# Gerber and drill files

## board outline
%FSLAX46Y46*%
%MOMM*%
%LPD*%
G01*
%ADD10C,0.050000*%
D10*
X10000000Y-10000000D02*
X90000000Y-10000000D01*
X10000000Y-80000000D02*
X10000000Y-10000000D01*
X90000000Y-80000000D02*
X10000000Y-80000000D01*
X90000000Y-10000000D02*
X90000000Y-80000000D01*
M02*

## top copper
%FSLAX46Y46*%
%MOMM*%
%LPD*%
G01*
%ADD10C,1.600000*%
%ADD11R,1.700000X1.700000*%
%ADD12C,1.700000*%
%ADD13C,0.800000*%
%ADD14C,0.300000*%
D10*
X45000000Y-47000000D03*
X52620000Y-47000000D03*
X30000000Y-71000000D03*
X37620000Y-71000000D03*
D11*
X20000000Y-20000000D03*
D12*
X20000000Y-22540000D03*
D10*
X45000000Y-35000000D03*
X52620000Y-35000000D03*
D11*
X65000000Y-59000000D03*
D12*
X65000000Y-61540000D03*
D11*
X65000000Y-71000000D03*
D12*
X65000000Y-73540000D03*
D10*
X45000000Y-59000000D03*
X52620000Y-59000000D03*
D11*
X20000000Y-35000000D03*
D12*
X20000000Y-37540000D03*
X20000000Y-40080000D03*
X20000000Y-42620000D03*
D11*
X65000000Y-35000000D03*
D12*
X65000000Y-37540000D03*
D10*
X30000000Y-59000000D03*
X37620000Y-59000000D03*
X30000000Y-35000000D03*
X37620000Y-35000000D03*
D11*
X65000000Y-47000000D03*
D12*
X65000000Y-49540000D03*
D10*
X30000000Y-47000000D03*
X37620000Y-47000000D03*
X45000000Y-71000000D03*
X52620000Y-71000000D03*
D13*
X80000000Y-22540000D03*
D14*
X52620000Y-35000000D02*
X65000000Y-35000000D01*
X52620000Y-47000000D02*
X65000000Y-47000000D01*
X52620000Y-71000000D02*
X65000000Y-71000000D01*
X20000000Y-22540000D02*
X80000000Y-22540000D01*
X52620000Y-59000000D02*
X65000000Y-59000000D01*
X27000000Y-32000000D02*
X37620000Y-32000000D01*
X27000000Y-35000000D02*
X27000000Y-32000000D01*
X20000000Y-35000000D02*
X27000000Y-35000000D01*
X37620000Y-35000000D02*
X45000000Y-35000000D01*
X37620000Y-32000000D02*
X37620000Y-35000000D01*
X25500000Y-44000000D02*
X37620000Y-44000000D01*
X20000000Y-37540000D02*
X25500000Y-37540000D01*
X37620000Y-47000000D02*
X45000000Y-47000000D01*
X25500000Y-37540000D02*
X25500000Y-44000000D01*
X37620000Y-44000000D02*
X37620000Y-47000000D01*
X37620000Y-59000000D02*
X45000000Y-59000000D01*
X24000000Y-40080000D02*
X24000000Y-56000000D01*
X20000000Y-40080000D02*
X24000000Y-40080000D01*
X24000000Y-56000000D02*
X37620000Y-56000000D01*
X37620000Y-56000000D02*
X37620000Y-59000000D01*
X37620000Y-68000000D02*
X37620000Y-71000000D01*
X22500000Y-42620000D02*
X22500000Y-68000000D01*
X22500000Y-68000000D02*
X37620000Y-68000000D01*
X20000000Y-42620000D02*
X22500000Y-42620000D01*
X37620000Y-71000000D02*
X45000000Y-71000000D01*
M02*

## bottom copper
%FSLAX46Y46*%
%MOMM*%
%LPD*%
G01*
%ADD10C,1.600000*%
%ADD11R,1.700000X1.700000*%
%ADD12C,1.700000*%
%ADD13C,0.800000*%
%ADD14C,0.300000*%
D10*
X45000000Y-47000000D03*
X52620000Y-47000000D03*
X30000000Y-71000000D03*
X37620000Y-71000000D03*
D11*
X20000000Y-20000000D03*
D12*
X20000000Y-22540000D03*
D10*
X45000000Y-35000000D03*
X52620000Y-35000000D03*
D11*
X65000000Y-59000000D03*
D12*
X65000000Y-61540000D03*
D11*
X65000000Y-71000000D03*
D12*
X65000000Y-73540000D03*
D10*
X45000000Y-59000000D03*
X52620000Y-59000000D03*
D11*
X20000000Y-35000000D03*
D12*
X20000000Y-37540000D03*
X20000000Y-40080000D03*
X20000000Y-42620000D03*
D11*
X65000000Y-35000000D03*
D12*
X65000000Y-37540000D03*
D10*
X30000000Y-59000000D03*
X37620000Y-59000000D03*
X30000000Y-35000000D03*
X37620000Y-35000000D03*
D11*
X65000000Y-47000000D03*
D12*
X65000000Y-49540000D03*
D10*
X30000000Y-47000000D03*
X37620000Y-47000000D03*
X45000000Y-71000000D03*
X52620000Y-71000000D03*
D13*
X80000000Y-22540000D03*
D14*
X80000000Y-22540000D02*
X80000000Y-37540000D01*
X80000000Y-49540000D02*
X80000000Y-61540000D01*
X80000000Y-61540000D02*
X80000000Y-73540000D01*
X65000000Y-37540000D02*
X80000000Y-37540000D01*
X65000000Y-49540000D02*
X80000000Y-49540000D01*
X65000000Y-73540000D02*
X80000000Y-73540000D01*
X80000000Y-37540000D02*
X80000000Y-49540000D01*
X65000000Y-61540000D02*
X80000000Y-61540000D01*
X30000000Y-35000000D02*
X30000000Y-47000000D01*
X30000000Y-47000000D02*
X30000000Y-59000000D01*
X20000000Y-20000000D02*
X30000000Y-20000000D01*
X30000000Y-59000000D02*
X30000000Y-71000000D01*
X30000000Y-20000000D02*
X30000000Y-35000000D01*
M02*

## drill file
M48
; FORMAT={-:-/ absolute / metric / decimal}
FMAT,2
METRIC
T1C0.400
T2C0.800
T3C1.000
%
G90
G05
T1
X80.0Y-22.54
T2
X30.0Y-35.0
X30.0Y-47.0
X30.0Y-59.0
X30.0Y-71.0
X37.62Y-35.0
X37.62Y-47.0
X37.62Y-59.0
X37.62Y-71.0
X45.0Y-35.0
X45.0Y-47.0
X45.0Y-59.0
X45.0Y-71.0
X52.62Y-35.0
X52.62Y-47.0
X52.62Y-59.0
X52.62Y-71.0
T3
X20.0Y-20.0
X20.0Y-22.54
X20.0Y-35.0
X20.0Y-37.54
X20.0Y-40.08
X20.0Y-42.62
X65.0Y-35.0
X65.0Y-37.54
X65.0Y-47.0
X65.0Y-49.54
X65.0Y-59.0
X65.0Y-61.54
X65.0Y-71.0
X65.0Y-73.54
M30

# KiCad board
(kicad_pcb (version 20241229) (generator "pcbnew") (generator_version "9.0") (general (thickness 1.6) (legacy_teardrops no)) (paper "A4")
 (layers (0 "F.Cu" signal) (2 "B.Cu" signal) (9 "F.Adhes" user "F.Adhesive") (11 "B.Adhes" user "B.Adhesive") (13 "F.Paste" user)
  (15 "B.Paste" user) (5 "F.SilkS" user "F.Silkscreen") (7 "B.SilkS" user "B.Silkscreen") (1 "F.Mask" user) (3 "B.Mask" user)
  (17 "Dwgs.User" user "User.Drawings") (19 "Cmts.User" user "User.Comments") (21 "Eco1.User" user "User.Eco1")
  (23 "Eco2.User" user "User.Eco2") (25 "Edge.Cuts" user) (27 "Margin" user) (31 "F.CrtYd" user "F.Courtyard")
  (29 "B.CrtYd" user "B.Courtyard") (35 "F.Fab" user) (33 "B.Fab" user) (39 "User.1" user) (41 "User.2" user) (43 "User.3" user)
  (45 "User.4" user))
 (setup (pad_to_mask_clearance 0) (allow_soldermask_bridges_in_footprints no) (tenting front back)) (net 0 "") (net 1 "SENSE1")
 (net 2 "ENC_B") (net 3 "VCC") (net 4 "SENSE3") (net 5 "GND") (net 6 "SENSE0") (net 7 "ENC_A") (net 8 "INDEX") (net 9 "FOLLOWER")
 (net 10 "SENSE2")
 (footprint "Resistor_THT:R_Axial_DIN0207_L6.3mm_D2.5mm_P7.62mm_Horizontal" (layer "F.Cu") (at 45 47)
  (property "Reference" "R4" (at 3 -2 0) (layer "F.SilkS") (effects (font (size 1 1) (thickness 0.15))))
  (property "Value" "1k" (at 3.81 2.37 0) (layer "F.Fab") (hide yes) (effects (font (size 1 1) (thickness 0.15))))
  (pad "1" thru_hole circle (at 0 0) (size 1.6 1.6) (drill 0.8) (layers "*.Cu" "*.Mask") (remove_unused_layers no) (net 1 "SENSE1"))
  (pad "2" thru_hole circle (at 7.62 0) (size 1.6 1.6) (drill 0.8) (layers "*.Cu" "*.Mask") (remove_unused_layers no) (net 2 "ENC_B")))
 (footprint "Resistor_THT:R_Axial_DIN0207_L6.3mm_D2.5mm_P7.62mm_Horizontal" (layer "F.Cu") (at 30 71)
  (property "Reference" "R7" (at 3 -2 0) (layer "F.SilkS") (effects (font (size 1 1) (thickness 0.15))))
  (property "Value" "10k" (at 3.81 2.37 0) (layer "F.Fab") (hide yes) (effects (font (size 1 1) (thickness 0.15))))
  (pad "1" thru_hole circle (at 0 0) (size 1.6 1.6) (drill 0.8) (layers "*.Cu" "*.Mask") (remove_unused_layers no) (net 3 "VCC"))
  (pad "2" thru_hole circle (at 7.62 0) (size 1.6 1.6) (drill 0.8) (layers "*.Cu" "*.Mask") (remove_unused_layers no) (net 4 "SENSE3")))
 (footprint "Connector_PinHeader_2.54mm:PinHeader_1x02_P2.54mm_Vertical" (layer "F.Cu") (at 20 20)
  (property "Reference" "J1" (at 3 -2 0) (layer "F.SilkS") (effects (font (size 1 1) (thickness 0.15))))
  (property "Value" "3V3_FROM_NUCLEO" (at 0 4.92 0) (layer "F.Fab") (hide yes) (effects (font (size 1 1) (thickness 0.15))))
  (pad "1" thru_hole rect (at 0 0) (size 1.7 1.7) (drill 1) (layers "*.Cu" "*.Mask") (remove_unused_layers no) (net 3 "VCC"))
  (pad "2" thru_hole circle (at 0 2.54) (size 1.7 1.7) (drill 1) (layers "*.Cu" "*.Mask") (remove_unused_layers no) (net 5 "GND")))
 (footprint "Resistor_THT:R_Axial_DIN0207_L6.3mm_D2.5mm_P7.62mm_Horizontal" (layer "F.Cu") (at 45 35)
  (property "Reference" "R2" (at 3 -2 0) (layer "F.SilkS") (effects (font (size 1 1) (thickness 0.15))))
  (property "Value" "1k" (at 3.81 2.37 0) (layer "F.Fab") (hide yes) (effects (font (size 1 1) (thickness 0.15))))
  (pad "1" thru_hole circle (at 0 0) (size 1.6 1.6) (drill 0.8) (layers "*.Cu" "*.Mask") (remove_unused_layers no) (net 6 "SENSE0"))
  (pad "2" thru_hole circle (at 7.62 0) (size 1.6 1.6) (drill 0.8) (layers "*.Cu" "*.Mask") (remove_unused_layers no) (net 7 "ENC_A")))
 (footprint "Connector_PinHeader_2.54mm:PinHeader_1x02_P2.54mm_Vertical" (layer "F.Cu") (at 65 59)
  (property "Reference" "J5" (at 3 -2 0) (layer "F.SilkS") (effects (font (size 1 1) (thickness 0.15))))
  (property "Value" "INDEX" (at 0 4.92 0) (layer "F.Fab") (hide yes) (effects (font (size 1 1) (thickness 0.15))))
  (pad "1" thru_hole rect (at 0 0) (size 1.7 1.7) (drill 1) (layers "*.Cu" "*.Mask") (remove_unused_layers no) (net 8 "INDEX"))
  (pad "2" thru_hole circle (at 0 2.54) (size 1.7 1.7) (drill 1) (layers "*.Cu" "*.Mask") (remove_unused_layers no) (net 5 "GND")))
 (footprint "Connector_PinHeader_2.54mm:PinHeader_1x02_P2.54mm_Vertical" (layer "F.Cu") (at 65 71)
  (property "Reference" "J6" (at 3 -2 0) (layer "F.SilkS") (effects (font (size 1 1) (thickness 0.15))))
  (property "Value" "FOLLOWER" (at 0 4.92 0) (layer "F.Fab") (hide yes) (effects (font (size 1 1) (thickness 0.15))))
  (pad "1" thru_hole rect (at 0 0) (size 1.7 1.7) (drill 1) (layers "*.Cu" "*.Mask") (remove_unused_layers no) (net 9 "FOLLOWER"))
  (pad "2" thru_hole circle (at 0 2.54) (size 1.7 1.7) (drill 1) (layers "*.Cu" "*.Mask") (remove_unused_layers no) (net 5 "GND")))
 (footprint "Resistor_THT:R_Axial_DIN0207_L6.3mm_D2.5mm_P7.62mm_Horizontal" (layer "F.Cu") (at 45 59)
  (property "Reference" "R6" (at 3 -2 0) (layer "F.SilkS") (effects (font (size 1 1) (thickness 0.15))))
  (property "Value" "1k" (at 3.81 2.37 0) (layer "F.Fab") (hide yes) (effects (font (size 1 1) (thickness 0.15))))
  (pad "1" thru_hole circle (at 0 0) (size 1.6 1.6) (drill 0.8) (layers "*.Cu" "*.Mask") (remove_unused_layers no) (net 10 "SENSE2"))
  (pad "2" thru_hole circle (at 7.62 0) (size 1.6 1.6) (drill 0.8) (layers "*.Cu" "*.Mask") (remove_unused_layers no) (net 8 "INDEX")))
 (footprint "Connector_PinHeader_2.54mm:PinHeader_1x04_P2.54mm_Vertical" (layer "F.Cu") (at 20 35)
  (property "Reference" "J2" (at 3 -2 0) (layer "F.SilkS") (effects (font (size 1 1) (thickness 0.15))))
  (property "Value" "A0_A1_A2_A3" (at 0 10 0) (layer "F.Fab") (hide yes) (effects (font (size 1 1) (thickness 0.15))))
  (pad "1" thru_hole rect (at 0 0) (size 1.7 1.7) (drill 1) (layers "*.Cu" "*.Mask") (remove_unused_layers no) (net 6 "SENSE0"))
  (pad "2" thru_hole circle (at 0 2.54) (size 1.7 1.7) (drill 1) (layers "*.Cu" "*.Mask") (remove_unused_layers no) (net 1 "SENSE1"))
  (pad "3" thru_hole circle (at 0 5.08) (size 1.7 1.7) (drill 1) (layers "*.Cu" "*.Mask") (remove_unused_layers no) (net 10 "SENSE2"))
  (pad "4" thru_hole circle (at 0 7.62) (size 1.7 1.7) (drill 1) (layers "*.Cu" "*.Mask") (remove_unused_layers no) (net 4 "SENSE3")))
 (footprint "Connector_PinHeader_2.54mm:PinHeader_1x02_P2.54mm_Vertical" (layer "F.Cu") (at 65 35)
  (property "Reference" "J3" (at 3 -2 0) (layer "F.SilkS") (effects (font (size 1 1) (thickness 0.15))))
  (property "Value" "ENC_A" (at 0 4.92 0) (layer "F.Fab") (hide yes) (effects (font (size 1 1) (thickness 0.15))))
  (pad "1" thru_hole rect (at 0 0) (size 1.7 1.7) (drill 1) (layers "*.Cu" "*.Mask") (remove_unused_layers no) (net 7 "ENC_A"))
  (pad "2" thru_hole circle (at 0 2.54) (size 1.7 1.7) (drill 1) (layers "*.Cu" "*.Mask") (remove_unused_layers no) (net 5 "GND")))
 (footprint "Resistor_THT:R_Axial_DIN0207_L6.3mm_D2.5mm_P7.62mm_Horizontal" (layer "F.Cu") (at 30 59)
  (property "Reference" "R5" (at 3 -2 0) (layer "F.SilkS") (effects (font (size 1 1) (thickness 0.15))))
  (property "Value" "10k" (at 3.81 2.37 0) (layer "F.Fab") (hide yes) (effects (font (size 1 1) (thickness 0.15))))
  (pad "1" thru_hole circle (at 0 0) (size 1.6 1.6) (drill 0.8) (layers "*.Cu" "*.Mask") (remove_unused_layers no) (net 3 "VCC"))
  (pad "2" thru_hole circle (at 7.62 0) (size 1.6 1.6) (drill 0.8) (layers "*.Cu" "*.Mask") (remove_unused_layers no) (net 10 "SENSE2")))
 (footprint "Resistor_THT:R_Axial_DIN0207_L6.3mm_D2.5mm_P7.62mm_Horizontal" (layer "F.Cu") (at 30 35)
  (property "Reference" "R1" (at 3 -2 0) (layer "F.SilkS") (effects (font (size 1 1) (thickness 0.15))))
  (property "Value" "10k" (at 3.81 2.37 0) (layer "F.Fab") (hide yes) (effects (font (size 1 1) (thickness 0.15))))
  (pad "1" thru_hole circle (at 0 0) (size 1.6 1.6) (drill 0.8) (layers "*.Cu" "*.Mask") (remove_unused_layers no) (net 3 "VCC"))
  (pad "2" thru_hole circle (at 7.62 0) (size 1.6 1.6) (drill 0.8) (layers "*.Cu" "*.Mask") (remove_unused_layers no) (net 6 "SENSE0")))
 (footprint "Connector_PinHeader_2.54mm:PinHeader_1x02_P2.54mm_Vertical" (layer "F.Cu") (at 65 47)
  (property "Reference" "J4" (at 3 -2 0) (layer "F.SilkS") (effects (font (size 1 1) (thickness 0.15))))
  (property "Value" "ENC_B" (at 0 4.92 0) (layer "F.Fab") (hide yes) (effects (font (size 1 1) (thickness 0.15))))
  (pad "1" thru_hole rect (at 0 0) (size 1.7 1.7) (drill 1) (layers "*.Cu" "*.Mask") (remove_unused_layers no) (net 2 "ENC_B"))
  (pad "2" thru_hole circle (at 0 2.54) (size 1.7 1.7) (drill 1) (layers "*.Cu" "*.Mask") (remove_unused_layers no) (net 5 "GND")))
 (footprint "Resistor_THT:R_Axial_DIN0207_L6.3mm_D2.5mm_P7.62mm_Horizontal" (layer "F.Cu") (at 30 47)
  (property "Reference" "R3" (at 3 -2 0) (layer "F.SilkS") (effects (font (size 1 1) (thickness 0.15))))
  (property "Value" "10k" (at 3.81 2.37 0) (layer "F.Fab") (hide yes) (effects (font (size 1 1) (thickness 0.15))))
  (pad "1" thru_hole circle (at 0 0) (size 1.6 1.6) (drill 0.8) (layers "*.Cu" "*.Mask") (remove_unused_layers no) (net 3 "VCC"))
  (pad "2" thru_hole circle (at 7.62 0) (size 1.6 1.6) (drill 0.8) (layers "*.Cu" "*.Mask") (remove_unused_layers no) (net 1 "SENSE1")))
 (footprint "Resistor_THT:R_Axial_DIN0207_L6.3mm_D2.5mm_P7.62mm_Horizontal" (layer "F.Cu") (at 45 71)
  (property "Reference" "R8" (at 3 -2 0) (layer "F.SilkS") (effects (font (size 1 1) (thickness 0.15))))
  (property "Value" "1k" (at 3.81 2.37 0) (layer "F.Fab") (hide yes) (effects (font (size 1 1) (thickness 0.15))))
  (pad "1" thru_hole circle (at 0 0) (size 1.6 1.6) (drill 0.8) (layers "*.Cu" "*.Mask") (remove_unused_layers no) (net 4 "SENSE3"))
  (pad "2" thru_hole circle (at 7.62 0) (size 1.6 1.6) (drill 0.8) (layers "*.Cu" "*.Mask") (remove_unused_layers no) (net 9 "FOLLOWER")))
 (gr_line (start 10 10) (end 90 10) (stroke (width 0.05) (type default)) (layer "Edge.Cuts"))
 (gr_line (start 10 80) (end 10 10) (stroke (width 0.05) (type default)) (layer "Edge.Cuts"))
 (gr_line (start 90 80) (end 10 80) (stroke (width 0.05) (type default)) (layer "Edge.Cuts"))
 (gr_line (start 90 10) (end 90 80) (stroke (width 0.05) (type default)) (layer "Edge.Cuts"))
 (segment (start 52.62 35) (end 65 35) (width 0.3) (layer "F.Cu") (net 7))
 (segment (start 52.62 47) (end 65 47) (width 0.3) (layer "F.Cu") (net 2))
 (segment (start 52.62 71) (end 65 71) (width 0.3) (layer "F.Cu") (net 9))
 (segment (start 20 22.54) (end 80 22.54) (width 0.3) (layer "F.Cu") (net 5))
 (via (at 80 22.54) (size 0.8) (drill 0.4) (layers "F.Cu" "B.Cu") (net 5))
 (segment (start 80 22.54) (end 80 37.54) (width 0.3) (layer "B.Cu") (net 5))
 (segment (start 80 49.54) (end 80 61.54) (width 0.3) (layer "B.Cu") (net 5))
 (segment (start 80 61.54) (end 80 73.54) (width 0.3) (layer "B.Cu") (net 5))
 (segment (start 65 37.54) (end 80 37.54) (width 0.3) (layer "B.Cu") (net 5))
 (segment (start 65 49.54) (end 80 49.54) (width 0.3) (layer "B.Cu") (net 5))
 (segment (start 65 73.54) (end 80 73.54) (width 0.3) (layer "B.Cu") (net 5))
 (segment (start 80 37.54) (end 80 49.54) (width 0.3) (layer "B.Cu") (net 5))
 (segment (start 65 61.54) (end 80 61.54) (width 0.3) (layer "B.Cu") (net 5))
 (segment (start 52.62 59) (end 65 59) (width 0.3) (layer "F.Cu") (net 8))
 (segment (start 27 32) (end 37.62 32) (width 0.3) (layer "F.Cu") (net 6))
 (segment (start 27 35) (end 27 32) (width 0.3) (layer "F.Cu") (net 6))
 (segment (start 20 35) (end 27 35) (width 0.3) (layer "F.Cu") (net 6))
 (segment (start 37.62 35) (end 45 35) (width 0.3) (layer "F.Cu") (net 6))
 (segment (start 37.62 32) (end 37.62 35) (width 0.3) (layer "F.Cu") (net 6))
 (segment (start 25.5 44) (end 37.62 44) (width 0.3) (layer "F.Cu") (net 1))
 (segment (start 20 37.54) (end 25.5 37.54) (width 0.3) (layer "F.Cu") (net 1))
 (segment (start 37.62 47) (end 45 47) (width 0.3) (layer "F.Cu") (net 1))
 (segment (start 25.5 37.54) (end 25.5 44) (width 0.3) (layer "F.Cu") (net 1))
 (segment (start 37.62 44) (end 37.62 47) (width 0.3) (layer "F.Cu") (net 1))
 (segment (start 37.62 59) (end 45 59) (width 0.3) (layer "F.Cu") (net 10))
 (segment (start 24 40.08) (end 24 56) (width 0.3) (layer "F.Cu") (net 10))
 (segment (start 20 40.08) (end 24 40.08) (width 0.3) (layer "F.Cu") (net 10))
 (segment (start 24 56) (end 37.62 56) (width 0.3) (layer "F.Cu") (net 10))
 (segment (start 37.62 56) (end 37.62 59) (width 0.3) (layer "F.Cu") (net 10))
 (segment (start 37.62 68) (end 37.62 71) (width 0.3) (layer "F.Cu") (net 4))
 (segment (start 22.5 42.62) (end 22.5 68) (width 0.3) (layer "F.Cu") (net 4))
 (segment (start 22.5 68) (end 37.62 68) (width 0.3) (layer "F.Cu") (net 4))
 (segment (start 20 42.62) (end 22.5 42.62) (width 0.3) (layer "F.Cu") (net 4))
 (segment (start 37.62 71) (end 45 71) (width 0.3) (layer "F.Cu") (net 4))
 (segment (start 30 35) (end 30 47) (width 0.3) (layer "B.Cu") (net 3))
 (segment (start 30 47) (end 30 59) (width 0.3) (layer "B.Cu") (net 3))
 (segment (start 20 20) (end 30 20) (width 0.3) (layer "B.Cu") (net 3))
 (segment (start 30 59) (end 30 71) (width 0.3) (layer "B.Cu") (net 3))
 (segment (start 30 20) (end 30 35) (width 0.3) (layer "B.Cu") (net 3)))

